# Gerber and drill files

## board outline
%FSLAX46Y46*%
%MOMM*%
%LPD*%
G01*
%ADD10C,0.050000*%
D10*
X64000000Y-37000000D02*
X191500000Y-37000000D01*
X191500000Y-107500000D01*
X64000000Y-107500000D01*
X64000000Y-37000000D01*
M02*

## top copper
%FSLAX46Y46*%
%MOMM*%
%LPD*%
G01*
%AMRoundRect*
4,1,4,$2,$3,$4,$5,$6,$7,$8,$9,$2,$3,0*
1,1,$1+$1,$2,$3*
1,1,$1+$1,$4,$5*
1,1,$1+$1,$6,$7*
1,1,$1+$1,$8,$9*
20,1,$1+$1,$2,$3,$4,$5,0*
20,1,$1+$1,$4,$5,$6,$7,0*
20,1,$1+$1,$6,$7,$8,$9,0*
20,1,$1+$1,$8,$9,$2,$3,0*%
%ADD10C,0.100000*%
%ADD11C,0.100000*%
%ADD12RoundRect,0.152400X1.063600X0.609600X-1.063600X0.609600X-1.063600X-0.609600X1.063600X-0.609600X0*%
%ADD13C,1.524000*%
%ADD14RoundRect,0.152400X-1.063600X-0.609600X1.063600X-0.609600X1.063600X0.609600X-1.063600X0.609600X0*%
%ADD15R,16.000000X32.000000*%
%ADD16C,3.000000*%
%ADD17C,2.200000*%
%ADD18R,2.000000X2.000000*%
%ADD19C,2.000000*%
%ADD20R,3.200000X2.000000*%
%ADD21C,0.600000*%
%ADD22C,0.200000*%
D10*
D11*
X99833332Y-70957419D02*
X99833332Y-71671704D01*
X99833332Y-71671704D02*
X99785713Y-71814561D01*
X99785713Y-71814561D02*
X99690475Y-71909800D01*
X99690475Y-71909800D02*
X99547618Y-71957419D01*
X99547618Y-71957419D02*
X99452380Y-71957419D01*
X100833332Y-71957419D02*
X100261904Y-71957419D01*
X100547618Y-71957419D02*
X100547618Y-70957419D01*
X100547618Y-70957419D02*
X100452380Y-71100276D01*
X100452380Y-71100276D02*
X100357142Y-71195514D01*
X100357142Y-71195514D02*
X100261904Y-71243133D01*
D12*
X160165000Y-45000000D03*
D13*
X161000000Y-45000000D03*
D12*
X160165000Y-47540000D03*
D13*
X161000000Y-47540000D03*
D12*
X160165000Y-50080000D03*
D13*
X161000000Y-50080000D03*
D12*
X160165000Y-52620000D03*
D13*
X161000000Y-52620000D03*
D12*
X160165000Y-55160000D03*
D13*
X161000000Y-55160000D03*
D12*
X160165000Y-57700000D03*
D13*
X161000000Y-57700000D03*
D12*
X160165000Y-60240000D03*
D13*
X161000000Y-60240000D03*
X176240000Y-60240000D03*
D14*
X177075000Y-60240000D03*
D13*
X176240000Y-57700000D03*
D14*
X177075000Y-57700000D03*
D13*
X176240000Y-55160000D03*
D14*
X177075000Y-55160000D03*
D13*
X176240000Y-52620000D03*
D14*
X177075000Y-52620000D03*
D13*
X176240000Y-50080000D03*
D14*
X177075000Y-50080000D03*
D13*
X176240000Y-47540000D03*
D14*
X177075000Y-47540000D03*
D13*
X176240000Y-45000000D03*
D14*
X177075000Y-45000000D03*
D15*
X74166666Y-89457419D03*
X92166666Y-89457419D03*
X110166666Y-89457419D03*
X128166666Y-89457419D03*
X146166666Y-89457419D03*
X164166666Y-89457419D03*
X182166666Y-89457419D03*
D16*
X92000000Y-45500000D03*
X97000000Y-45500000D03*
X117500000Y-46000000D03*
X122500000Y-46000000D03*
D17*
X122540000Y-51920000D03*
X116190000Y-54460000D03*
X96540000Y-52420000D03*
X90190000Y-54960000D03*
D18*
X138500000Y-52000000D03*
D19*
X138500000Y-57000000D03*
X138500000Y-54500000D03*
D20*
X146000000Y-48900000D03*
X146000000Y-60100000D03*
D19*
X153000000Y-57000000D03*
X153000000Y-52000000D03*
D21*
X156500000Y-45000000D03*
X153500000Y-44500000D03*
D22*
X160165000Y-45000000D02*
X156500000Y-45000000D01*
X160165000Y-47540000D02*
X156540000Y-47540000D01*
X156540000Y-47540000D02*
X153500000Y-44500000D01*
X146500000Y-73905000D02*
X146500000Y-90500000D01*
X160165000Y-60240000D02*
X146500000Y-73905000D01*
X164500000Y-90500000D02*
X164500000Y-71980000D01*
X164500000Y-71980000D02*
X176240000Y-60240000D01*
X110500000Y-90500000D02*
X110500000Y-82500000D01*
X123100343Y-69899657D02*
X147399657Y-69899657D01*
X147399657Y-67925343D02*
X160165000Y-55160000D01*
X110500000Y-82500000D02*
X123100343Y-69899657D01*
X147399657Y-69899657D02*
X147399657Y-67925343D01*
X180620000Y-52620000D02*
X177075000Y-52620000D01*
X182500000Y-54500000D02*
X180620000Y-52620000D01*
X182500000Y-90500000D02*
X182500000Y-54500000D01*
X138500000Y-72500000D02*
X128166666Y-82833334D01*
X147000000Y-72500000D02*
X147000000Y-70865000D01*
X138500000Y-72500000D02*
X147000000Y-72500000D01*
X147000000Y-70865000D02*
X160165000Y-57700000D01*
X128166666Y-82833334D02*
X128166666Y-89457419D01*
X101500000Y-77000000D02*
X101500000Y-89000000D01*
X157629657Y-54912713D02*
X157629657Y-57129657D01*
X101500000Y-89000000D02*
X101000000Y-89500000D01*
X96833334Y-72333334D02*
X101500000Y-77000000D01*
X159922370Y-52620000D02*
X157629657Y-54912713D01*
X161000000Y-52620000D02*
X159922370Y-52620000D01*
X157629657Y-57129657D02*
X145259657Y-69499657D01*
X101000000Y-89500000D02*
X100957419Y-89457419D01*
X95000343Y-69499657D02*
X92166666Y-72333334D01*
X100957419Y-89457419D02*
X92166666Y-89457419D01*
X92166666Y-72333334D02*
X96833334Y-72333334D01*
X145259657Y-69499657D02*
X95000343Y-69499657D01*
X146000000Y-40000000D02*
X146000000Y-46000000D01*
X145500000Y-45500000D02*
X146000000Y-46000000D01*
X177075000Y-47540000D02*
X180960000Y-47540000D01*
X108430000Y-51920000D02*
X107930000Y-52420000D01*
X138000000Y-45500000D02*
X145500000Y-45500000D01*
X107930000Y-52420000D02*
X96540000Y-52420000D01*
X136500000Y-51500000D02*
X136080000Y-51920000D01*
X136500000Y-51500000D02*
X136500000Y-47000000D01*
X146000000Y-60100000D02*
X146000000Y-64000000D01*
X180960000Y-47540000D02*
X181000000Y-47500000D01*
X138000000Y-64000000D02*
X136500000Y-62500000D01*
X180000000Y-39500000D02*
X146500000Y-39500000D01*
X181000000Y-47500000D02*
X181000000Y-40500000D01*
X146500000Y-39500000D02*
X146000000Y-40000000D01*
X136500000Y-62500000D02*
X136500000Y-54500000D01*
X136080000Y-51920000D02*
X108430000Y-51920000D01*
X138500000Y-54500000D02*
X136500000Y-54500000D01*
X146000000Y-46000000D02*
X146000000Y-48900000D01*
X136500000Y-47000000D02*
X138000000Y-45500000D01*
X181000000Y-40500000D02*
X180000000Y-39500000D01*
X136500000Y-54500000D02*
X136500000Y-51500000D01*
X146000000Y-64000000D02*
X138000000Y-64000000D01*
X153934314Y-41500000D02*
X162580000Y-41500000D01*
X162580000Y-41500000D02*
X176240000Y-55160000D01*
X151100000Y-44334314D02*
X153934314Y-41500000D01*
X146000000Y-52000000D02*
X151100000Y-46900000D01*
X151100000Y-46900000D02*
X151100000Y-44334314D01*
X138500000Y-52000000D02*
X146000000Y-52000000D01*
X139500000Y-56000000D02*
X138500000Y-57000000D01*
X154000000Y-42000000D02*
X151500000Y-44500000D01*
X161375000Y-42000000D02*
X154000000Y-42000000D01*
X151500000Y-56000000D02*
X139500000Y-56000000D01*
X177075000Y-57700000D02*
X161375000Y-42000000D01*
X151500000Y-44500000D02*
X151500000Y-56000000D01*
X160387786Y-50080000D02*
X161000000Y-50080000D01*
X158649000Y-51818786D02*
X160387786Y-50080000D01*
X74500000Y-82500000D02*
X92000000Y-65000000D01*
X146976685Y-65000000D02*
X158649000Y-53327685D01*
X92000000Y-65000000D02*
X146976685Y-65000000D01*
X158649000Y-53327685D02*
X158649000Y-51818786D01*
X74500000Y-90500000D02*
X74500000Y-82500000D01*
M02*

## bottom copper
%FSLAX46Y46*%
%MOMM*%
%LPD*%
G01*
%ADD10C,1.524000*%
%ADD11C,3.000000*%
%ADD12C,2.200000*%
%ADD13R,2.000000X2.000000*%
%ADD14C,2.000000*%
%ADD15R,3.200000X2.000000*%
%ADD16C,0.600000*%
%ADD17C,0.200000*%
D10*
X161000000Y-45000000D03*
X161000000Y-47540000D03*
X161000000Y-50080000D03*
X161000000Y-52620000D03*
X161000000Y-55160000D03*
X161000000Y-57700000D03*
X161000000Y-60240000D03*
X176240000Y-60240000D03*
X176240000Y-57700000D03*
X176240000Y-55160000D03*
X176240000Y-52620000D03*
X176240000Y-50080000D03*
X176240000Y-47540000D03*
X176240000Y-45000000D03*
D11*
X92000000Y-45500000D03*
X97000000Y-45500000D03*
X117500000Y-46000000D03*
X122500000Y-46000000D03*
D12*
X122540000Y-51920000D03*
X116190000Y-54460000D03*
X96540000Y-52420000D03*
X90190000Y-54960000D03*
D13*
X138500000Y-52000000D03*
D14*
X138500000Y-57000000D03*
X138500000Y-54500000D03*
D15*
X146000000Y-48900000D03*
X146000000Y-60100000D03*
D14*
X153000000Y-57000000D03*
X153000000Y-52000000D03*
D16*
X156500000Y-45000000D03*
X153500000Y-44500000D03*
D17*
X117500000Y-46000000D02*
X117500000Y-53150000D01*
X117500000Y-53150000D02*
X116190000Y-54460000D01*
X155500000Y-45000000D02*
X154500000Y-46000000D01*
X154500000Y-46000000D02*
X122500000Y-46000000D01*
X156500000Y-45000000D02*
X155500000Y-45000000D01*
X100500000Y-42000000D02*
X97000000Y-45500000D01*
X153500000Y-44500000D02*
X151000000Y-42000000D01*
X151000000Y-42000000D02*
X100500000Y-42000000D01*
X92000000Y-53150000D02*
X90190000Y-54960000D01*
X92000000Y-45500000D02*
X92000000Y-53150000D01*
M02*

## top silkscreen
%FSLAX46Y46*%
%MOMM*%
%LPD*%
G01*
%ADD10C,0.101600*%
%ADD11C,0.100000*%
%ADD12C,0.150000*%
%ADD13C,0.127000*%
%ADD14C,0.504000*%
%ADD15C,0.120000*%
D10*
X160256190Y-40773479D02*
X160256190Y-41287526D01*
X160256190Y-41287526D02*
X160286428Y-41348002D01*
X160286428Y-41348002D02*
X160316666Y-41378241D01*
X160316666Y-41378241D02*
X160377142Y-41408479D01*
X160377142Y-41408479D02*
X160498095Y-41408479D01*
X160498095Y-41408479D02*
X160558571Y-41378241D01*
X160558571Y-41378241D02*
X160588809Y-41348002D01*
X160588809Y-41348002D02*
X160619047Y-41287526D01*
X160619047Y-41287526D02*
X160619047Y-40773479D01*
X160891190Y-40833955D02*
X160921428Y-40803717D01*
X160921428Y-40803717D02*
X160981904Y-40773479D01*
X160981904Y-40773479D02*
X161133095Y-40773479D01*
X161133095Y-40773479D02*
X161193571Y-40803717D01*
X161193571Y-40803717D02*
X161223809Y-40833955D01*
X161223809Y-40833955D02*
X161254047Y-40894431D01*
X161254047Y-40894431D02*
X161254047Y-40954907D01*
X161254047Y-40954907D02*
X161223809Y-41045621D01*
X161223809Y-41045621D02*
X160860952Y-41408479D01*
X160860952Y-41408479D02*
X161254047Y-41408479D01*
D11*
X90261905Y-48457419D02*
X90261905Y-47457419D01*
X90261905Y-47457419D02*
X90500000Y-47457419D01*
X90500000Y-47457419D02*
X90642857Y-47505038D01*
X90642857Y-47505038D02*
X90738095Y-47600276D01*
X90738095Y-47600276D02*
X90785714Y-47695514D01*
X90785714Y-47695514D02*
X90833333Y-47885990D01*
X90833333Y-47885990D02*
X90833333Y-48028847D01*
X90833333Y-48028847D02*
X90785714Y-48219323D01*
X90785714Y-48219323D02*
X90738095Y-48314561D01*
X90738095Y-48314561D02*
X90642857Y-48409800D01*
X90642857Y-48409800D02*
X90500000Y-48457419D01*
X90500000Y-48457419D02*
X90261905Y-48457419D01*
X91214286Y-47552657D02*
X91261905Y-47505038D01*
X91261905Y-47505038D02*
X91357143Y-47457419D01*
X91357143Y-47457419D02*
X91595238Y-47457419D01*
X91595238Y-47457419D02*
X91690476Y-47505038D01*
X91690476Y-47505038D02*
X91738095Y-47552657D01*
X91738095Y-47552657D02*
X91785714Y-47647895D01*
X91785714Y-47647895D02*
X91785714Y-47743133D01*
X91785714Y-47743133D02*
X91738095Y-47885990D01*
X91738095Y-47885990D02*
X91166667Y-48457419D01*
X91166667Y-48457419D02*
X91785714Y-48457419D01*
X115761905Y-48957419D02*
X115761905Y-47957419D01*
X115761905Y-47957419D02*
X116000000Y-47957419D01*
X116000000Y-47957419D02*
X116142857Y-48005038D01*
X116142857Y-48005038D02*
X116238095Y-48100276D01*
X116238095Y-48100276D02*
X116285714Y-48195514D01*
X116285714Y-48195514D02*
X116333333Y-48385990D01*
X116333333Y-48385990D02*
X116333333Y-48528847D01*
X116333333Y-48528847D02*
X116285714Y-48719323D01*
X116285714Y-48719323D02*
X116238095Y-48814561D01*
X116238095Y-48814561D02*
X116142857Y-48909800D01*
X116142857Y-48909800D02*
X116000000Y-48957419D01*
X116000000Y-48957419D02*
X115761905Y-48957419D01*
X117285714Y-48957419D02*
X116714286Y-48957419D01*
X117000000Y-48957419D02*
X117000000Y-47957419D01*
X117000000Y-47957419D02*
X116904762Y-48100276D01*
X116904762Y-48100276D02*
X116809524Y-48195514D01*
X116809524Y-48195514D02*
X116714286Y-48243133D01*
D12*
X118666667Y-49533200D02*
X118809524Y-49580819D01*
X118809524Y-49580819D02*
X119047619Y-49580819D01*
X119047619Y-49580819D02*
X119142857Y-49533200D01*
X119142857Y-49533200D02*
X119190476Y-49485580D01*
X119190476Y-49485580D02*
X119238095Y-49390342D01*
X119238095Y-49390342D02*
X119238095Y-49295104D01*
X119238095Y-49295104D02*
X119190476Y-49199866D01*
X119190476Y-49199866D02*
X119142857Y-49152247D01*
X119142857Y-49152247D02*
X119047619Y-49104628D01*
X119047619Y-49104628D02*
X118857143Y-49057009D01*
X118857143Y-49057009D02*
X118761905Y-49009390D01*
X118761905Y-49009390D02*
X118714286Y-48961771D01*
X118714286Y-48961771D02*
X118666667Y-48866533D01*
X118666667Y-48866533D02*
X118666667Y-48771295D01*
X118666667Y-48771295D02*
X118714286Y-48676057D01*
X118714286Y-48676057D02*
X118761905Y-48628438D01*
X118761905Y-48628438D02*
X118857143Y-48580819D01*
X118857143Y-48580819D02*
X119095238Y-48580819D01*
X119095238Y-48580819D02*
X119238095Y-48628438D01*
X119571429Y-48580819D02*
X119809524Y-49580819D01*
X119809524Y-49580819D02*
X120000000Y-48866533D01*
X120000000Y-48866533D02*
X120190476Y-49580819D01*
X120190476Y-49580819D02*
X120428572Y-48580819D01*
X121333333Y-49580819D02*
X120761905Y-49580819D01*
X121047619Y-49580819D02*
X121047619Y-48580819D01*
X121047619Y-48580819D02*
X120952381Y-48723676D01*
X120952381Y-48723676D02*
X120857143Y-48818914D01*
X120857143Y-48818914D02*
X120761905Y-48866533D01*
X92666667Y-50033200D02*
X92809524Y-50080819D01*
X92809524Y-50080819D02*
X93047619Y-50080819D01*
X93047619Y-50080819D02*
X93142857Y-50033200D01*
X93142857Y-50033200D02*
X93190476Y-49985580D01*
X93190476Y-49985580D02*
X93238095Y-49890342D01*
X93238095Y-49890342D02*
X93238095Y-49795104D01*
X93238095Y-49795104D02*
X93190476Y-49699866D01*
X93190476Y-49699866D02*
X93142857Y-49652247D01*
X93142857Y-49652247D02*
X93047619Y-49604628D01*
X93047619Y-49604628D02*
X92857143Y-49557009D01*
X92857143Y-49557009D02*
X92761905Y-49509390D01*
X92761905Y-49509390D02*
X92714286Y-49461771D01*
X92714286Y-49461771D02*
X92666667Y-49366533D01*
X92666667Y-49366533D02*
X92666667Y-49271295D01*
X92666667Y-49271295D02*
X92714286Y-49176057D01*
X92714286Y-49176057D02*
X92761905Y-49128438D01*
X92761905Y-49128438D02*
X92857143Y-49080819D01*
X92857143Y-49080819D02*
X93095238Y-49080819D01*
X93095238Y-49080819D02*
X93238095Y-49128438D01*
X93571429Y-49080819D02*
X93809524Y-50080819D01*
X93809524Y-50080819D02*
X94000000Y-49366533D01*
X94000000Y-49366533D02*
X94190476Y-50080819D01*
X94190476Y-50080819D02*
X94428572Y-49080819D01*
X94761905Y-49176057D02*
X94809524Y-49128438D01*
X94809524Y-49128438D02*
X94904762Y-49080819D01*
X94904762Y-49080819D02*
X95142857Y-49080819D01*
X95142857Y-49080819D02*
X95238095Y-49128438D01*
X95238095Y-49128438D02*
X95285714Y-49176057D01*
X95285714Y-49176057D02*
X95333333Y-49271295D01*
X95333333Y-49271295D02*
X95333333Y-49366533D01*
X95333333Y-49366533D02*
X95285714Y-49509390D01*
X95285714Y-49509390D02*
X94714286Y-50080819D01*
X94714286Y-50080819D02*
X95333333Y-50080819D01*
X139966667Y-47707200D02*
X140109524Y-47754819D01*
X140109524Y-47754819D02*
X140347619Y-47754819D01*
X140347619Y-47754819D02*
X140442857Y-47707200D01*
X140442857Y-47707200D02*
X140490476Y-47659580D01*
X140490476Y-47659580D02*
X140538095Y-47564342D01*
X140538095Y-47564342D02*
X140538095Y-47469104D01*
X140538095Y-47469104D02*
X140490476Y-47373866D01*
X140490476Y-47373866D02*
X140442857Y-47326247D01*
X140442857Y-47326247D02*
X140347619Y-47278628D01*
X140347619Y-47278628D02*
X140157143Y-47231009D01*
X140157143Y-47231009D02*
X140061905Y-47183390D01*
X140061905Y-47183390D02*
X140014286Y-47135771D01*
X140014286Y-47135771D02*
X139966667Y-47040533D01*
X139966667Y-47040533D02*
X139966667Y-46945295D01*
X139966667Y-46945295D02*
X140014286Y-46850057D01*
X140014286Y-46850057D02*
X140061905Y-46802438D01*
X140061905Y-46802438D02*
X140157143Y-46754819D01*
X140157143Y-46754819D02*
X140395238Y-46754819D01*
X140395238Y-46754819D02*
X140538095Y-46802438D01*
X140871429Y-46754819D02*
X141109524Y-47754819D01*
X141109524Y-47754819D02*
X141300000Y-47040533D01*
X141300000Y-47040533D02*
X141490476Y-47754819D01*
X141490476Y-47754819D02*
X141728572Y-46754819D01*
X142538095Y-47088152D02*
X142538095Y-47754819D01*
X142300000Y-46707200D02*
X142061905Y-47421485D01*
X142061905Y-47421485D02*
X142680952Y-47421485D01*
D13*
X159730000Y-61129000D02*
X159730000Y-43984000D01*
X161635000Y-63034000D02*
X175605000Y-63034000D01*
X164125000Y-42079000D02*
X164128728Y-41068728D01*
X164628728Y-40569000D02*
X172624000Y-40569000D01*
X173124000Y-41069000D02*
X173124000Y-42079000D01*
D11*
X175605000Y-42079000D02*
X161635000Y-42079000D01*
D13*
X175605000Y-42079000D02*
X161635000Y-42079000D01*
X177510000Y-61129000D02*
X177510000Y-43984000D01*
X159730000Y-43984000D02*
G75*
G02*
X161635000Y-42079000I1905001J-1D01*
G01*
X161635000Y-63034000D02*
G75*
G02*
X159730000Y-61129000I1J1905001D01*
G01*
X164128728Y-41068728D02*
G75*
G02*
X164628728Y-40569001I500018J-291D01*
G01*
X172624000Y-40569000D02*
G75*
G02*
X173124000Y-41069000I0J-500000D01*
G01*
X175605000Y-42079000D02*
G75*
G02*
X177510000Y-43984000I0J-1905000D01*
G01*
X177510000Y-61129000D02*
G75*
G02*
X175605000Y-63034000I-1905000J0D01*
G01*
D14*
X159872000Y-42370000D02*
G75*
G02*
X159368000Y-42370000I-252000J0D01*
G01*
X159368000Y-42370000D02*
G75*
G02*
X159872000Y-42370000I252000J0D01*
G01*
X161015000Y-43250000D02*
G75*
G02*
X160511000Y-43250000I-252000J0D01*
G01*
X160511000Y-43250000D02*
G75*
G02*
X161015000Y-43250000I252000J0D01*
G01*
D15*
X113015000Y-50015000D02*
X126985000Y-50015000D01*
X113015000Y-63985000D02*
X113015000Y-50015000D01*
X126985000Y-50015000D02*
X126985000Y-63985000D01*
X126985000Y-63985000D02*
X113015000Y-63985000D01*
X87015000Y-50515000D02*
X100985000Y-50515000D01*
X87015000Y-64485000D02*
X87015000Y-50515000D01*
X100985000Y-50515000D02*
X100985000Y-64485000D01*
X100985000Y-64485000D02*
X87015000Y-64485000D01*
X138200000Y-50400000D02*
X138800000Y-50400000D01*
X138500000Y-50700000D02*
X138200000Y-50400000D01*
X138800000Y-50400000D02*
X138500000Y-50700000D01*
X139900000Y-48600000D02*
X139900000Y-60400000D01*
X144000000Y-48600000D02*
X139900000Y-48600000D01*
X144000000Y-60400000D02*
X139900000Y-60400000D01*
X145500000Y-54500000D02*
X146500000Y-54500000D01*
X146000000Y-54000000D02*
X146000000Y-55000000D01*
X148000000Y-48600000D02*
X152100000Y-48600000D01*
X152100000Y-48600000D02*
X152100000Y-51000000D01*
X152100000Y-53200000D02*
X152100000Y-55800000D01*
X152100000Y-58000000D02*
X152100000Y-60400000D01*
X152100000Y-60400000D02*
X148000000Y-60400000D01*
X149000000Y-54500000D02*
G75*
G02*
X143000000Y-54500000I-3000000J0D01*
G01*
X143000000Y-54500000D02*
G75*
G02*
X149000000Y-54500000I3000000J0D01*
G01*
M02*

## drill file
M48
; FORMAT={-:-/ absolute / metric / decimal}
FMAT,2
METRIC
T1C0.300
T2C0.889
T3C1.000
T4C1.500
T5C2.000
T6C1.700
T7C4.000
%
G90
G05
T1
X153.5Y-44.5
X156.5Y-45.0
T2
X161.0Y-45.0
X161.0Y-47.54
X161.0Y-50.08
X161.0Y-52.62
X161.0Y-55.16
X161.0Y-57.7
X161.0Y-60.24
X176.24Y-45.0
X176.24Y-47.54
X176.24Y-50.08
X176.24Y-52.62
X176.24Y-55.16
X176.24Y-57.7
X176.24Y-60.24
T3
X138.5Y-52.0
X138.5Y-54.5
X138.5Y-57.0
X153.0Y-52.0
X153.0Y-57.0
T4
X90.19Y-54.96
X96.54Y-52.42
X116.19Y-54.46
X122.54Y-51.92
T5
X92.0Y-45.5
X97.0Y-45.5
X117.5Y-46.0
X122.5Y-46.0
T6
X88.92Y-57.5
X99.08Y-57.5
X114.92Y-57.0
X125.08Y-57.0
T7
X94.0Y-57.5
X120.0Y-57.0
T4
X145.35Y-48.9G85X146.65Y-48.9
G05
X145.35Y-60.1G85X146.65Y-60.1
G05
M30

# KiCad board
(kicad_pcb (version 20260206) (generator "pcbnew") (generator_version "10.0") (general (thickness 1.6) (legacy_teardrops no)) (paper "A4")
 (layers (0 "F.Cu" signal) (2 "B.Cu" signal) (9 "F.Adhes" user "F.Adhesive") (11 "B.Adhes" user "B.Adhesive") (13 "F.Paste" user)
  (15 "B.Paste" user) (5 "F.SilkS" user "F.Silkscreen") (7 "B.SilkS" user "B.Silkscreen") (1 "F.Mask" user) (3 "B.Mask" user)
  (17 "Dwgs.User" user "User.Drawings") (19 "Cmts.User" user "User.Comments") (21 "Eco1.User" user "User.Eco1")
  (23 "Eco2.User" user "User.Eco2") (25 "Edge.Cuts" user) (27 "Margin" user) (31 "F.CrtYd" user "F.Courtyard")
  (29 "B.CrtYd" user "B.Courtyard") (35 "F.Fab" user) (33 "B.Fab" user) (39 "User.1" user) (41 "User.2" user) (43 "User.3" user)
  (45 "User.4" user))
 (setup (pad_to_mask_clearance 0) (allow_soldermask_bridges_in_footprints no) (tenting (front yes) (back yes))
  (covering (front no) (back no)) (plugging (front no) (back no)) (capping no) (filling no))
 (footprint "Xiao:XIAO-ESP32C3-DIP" (layer "F.Cu") (at 168.74 52.62)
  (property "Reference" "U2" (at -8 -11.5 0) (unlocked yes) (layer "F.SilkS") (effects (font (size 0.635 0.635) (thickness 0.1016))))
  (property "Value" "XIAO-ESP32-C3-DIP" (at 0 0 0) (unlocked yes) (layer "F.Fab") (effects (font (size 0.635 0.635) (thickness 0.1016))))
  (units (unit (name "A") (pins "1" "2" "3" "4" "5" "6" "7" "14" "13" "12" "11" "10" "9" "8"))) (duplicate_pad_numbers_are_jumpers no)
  (fp_line (start -9.01 8.509) (end -9.01 -8.636) (stroke (width 0.127) (type solid)) (layer "F.SilkS"))
  (fp_line (start -7.105 10.414) (end 6.865 10.414) (stroke (width 0.127) (type solid)) (layer "F.SilkS"))
  (fp_line (start -4.615 -10.541) (end -4.611272 -11.551272) (stroke (width 0.127) (type solid)) (layer "F.SilkS"))
  (fp_line (start -4.111272 -12.051) (end 3.884 -12.051) (stroke (width 0.127) (type solid)) (layer "F.SilkS"))
  (fp_line (start 4.384 -11.551) (end 4.384 -10.541) (stroke (width 0.127) (type solid)) (layer "F.SilkS"))
  (fp_line (start 6.865 -10.541) (end -7.105 -10.541) (stroke (width 0.1) (type solid)) (layer "F.SilkS"))
  (fp_line (start 6.865 -10.541) (end -7.105 -10.541) (stroke (width 0.127) (type solid)) (layer "F.SilkS"))
  (fp_line (start 8.77 8.509) (end 8.77 -8.636) (stroke (width 0.127) (type solid)) (layer "F.SilkS"))
  (fp_arc (start -9.01 -8.636) (mid -8.452038 -9.983038) (end -7.105 -10.541) (stroke (width 0.127) (type solid)) (layer "F.SilkS"))
  (fp_arc (start -7.105 10.414) (mid -8.452038 9.856038) (end -9.01 8.509) (stroke (width 0.127) (type solid)) (layer "F.SilkS"))
  (fp_arc (start -4.611272 -11.551272) (mid -4.464728 -11.90464) (end -4.111272 -12.051) (stroke (width 0.127) (type default))
   (layer "F.SilkS"))
  (fp_arc (start 3.884 -12.051) (mid 4.237553 -11.904553) (end 4.384 -11.551) (stroke (width 0.127) (type default)) (layer "F.SilkS"))
  (fp_arc (start 6.865 -10.541) (mid 8.212038 -9.983038) (end 8.77 -8.636) (stroke (width 0.127) (type solid)) (layer "F.SilkS"))
  (fp_arc (start 8.77 8.509) (mid 8.212038 9.856038) (end 6.865 10.414) (stroke (width 0.127) (type solid)) (layer "F.SilkS"))
  (fp_circle (center -9.12 -10.25) (end -9.12 -10.504) (stroke (width 0.5) (type solid)) (fill yes) (layer "F.SilkS"))
  (fp_circle (center -7.977 -9.37) (end -7.977 -9.624) (stroke (width 0.5) (type solid)) (fill yes) (layer "F.SilkS"))
  (pad "1" smd roundrect (at -8.575 -7.62 180) (size 2.432 1.524) (layers "F.Cu" "F.Mask") (roundrect_rratio 0.1) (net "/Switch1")
   (thermal_bridge_angle 45))
  (pad "1" thru_hole circle (at -7.74 -7.62 180) (size 1.524 1.524) (drill 0.889) (layers "*.Cu" "*.Mask") (remove_unused_layers no)
   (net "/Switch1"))
  (pad "2" smd roundrect (at -8.575 -5.08 180) (size 2.432 1.524) (layers "F.Cu" "F.Mask") (roundrect_rratio 0.1) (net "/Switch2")
   (thermal_bridge_angle 45))
  (pad "2" thru_hole circle (at -7.74 -5.08 180) (size 1.524 1.524) (drill 0.889) (layers "*.Cu" "*.Mask") (remove_unused_layers no)
   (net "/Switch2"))
  (pad "3" smd roundrect (at -8.575 -2.54 180) (size 2.432 1.524) (layers "F.Cu" "F.Mask") (roundrect_rratio 0.1) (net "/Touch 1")
   (thermal_bridge_angle 45))
  (pad "3" thru_hole circle (at -7.74 -2.54 180) (size 1.524 1.524) (drill 0.889) (layers "*.Cu" "*.Mask") (remove_unused_layers no)
   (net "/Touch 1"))
  (pad "4" smd roundrect (at -8.575 0 180) (size 2.432 1.524) (layers "F.Cu" "F.Mask") (roundrect_rratio 0.1) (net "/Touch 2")
   (thermal_bridge_angle 45))
  (pad "4" thru_hole circle (at -7.74 0 180) (size 1.524 1.524) (drill 0.889) (layers "*.Cu" "*.Mask") (remove_unused_layers no)
   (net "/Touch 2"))
  (pad "5" smd roundrect (at -8.575 2.54 180) (size 2.432 1.524) (layers "F.Cu" "F.Mask") (roundrect_rratio 0.1) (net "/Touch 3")
   (thermal_bridge_angle 45))
  (pad "5" thru_hole circle (at -7.74 2.54 180) (size 1.524 1.524) (drill 0.889) (layers "*.Cu" "*.Mask") (remove_unused_layers no)
   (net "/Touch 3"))
  (pad "6" smd roundrect (at -8.575 5.08 180) (size 2.432 1.524) (layers "F.Cu" "F.Mask") (roundrect_rratio 0.1) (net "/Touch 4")
   (thermal_bridge_angle 45))
  (pad "6" thru_hole circle (at -7.74 5.08 180) (size 1.524 1.524) (drill 0.889) (layers "*.Cu" "*.Mask") (remove_unused_layers no)
   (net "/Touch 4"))
  (pad "7" smd roundrect (at -8.575 7.62 180) (size 2.432 1.524) (layers "F.Cu" "F.Mask") (roundrect_rratio 0.1) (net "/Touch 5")
   (thermal_bridge_angle 45))
  (pad "7" thru_hole circle (at -7.74 7.62 180) (size 1.524 1.524) (drill 0.889) (layers "*.Cu" "*.Mask") (remove_unused_layers no)
   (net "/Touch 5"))
  (pad "8" thru_hole circle (at 7.5 7.62) (size 1.524 1.524) (drill 0.889) (layers "*.Cu" "*.Mask") (remove_unused_layers no)
   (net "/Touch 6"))
  (pad "8" smd roundrect (at 8.335 7.62) (size 2.432 1.524) (layers "F.Cu" "F.Mask") (roundrect_rratio 0.1) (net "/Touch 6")
   (thermal_bridge_angle 45))
  (pad "9" thru_hole circle (at 7.5 5.08) (size 1.524 1.524) (drill 0.889) (layers "*.Cu" "*.Mask") (remove_unused_layers no)
   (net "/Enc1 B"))
  (pad "9" smd roundrect (at 8.335 5.08) (size 2.432 1.524) (layers "F.Cu" "F.Mask") (roundrect_rratio 0.1) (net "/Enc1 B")
   (thermal_bridge_angle 45))
  (pad "10" thru_hole circle (at 7.5 2.54) (size 1.524 1.524) (drill 0.889) (layers "*.Cu" "*.Mask") (remove_unused_layers no)
   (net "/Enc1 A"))
  (pad "10" smd roundrect (at 8.335 2.54) (size 2.432 1.524) (layers "F.Cu" "F.Mask") (roundrect_rratio 0.1) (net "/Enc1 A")
   (thermal_bridge_angle 45))
  (pad "11" thru_hole circle (at 7.5 0) (size 1.524 1.524) (drill 0.889) (layers "*.Cu" "*.Mask") (remove_unused_layers no) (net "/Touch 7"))
  (pad "11" smd roundrect (at 8.335 0) (size 2.432 1.524) (layers "F.Cu" "F.Mask") (roundrect_rratio 0.1) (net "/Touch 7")
   (thermal_bridge_angle 45))
  (pad "12" thru_hole circle (at 7.5 -2.54) (size 1.524 1.524) (drill 0.889) (layers "*.Cu" "*.Mask") (remove_unused_layers no) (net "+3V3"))
  (pad "12" smd roundrect (at 8.335 -2.54) (size 2.432 1.524) (layers "F.Cu" "F.Mask") (roundrect_rratio 0.1) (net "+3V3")
   (thermal_bridge_angle 45))
  (pad "13" thru_hole circle (at 7.5 -5.08) (size 1.524 1.524) (drill 0.889) (layers "*.Cu" "*.Mask") (remove_unused_layers no) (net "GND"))
  (pad "13" smd roundrect (at 8.335 -5.08) (size 2.432 1.524) (layers "F.Cu" "F.Mask") (roundrect_rratio 0.1) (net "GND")
   (thermal_bridge_angle 45))
  (pad "14" thru_hole circle (at 7.5 -7.62) (size 1.524 1.524) (drill 0.889) (layers "*.Cu" "*.Mask") (remove_unused_layers no)
   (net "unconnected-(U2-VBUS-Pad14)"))
  (pad "14" smd roundrect (at 8.335 -7.62) (size 2.432 1.524) (layers "F.Cu" "F.Mask") (roundrect_rratio 0.1)
   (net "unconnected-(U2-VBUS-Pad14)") (thermal_bridge_angle 45)))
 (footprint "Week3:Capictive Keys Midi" (layer "F.Cu") (at 93.166666 89.457419)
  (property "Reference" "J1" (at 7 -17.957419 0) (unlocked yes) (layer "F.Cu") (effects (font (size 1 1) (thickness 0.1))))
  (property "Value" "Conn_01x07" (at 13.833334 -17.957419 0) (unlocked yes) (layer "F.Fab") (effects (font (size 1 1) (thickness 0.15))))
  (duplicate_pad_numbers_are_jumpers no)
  (pad "1" smd rect (at -19 0) (size 16 32) (layers "F.Cu" "F.Mask") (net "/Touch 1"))
  (pad "2" smd rect (at -1 0) (size 16 32) (layers "F.Cu" "F.Mask") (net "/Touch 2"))
  (pad "3" smd rect (at 17 0) (size 16 32) (layers "F.Cu" "F.Mask") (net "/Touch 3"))
  (pad "4" smd rect (at 35 0) (size 16 32) (layers "F.Cu" "F.Mask") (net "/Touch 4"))
  (pad "5" smd rect (at 53 0) (size 16 32) (layers "F.Cu" "F.Mask") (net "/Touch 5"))
  (pad "6" smd rect (at 71 0) (size 16 32) (layers "F.Cu" "F.Mask") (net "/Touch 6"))
  (pad "7" smd rect (at 89 0) (size 16 32) (layers "F.Cu" "F.Mask") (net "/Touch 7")))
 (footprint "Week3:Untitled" (layer "F.Cu") (at 91 48.5)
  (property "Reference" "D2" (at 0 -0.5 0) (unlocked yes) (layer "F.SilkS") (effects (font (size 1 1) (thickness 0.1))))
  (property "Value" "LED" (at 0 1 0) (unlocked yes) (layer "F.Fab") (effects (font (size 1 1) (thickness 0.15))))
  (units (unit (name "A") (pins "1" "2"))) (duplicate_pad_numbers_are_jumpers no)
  (pad "1" thru_hole circle (at 1 -3) (size 3 3) (drill 2) (layers "*.Cu" "*.Mask") (remove_unused_layers no) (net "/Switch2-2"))
  (pad "2" thru_hole circle (at 6 -3) (size 3 3) (drill 2) (layers "*.Cu" "*.Mask") (remove_unused_layers no) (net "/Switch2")))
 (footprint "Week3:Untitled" (layer "F.Cu") (at 116.5 49)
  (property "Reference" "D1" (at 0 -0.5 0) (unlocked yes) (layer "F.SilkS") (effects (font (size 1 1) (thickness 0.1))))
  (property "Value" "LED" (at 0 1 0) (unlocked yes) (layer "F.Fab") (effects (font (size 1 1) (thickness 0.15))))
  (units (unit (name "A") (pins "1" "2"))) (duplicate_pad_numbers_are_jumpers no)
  (pad "1" thru_hole circle (at 1 -3) (size 3 3) (drill 2) (layers "*.Cu" "*.Mask") (remove_unused_layers no) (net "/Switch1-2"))
  (pad "2" thru_hole circle (at 6 -3) (size 3 3) (drill 2) (layers "*.Cu" "*.Mask") (remove_unused_layers no) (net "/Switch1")))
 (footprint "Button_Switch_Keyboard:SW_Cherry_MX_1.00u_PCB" (layer "F.Cu") (at 122.54 51.92)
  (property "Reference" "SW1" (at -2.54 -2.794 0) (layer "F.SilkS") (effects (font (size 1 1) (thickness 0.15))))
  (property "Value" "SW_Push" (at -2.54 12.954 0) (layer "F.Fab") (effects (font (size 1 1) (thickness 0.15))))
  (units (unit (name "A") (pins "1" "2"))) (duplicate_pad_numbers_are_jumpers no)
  (fp_line (start -9.525 -1.905) (end 4.445 -1.905) (stroke (width 0.12) (type solid)) (layer "F.SilkS"))
  (fp_line (start -9.525 12.065) (end -9.525 -1.905) (stroke (width 0.12) (type solid)) (layer "F.SilkS"))
  (fp_line (start 4.445 -1.905) (end 4.445 12.065) (stroke (width 0.12) (type solid)) (layer "F.SilkS"))
  (fp_line (start 4.445 12.065) (end -9.525 12.065) (stroke (width 0.12) (type solid)) (layer "F.SilkS"))
  (pad "" np_thru_hole circle (at -7.62 5.08) (size 1.7 1.7) (drill 1.7) (layers "*.Cu" "*.Mask"))
  (pad "" np_thru_hole circle (at -2.54 5.08) (size 4 4) (drill 4) (layers "*.Cu" "*.Mask"))
  (pad "" np_thru_hole circle (at 2.54 5.08) (size 1.7 1.7) (drill 1.7) (layers "*.Cu" "*.Mask"))
  (pad "1" thru_hole circle (at 0 0) (size 2.2 2.2) (drill 1.5) (layers "*.Cu" "*.Mask") (remove_unused_layers no) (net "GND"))
  (pad "2" thru_hole circle (at -6.35 2.54) (size 2.2 2.2) (drill 1.5) (layers "*.Cu" "*.Mask") (remove_unused_layers no) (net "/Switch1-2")))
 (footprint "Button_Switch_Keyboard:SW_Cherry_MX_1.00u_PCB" (layer "F.Cu") (at 96.54 52.42)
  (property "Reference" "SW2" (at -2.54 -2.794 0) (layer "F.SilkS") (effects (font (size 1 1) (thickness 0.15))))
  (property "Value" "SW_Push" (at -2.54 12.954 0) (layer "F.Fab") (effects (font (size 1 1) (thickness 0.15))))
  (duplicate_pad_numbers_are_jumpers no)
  (fp_line (start -9.525 -1.905) (end 4.445 -1.905) (stroke (width 0.12) (type solid)) (layer "F.SilkS"))
  (fp_line (start -9.525 12.065) (end -9.525 -1.905) (stroke (width 0.12) (type solid)) (layer "F.SilkS"))
  (fp_line (start 4.445 -1.905) (end 4.445 12.065) (stroke (width 0.12) (type solid)) (layer "F.SilkS"))
  (fp_line (start 4.445 12.065) (end -9.525 12.065) (stroke (width 0.12) (type solid)) (layer "F.SilkS"))
  (pad "" np_thru_hole circle (at -7.62 5.08) (size 1.7 1.7) (drill 1.7) (layers "*.Cu" "*.Mask"))
  (pad "" np_thru_hole circle (at -2.54 5.08) (size 4 4) (drill 4) (layers "*.Cu" "*.Mask"))
  (pad "" np_thru_hole circle (at 2.54 5.08) (size 1.7 1.7) (drill 1.7) (layers "*.Cu" "*.Mask"))
  (pad "1" thru_hole circle (at 0 0) (size 2.2 2.2) (drill 1.5) (layers "*.Cu" "*.Mask") (remove_unused_layers no) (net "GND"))
  (pad "2" thru_hole circle (at -6.35 2.54) (size 2.2 2.2) (drill 1.5) (layers "*.Cu" "*.Mask") (remove_unused_layers no) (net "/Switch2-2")))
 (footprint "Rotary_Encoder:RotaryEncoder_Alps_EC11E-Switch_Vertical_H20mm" (layer "F.Cu") (at 138.5 52)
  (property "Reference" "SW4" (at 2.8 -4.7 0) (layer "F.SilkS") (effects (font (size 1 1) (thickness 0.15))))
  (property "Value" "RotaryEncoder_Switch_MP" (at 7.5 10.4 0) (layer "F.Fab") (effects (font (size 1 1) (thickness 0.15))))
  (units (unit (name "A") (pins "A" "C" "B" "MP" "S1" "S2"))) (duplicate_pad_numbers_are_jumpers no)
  (fp_line (start -0.3 -1.6) (end 0.3 -1.6) (stroke (width 0.12) (type solid)) (layer "F.SilkS"))
  (fp_line (start 0 -1.3) (end -0.3 -1.6) (stroke (width 0.12) (type solid)) (layer "F.SilkS"))
  (fp_line (start 0.3 -1.6) (end 0 -1.3) (stroke (width 0.12) (type solid)) (layer "F.SilkS"))
  (fp_line (start 1.4 -3.4) (end 1.4 8.4) (stroke (width 0.12) (type solid)) (layer "F.SilkS"))
  (fp_line (start 5.5 -3.4) (end 1.4 -3.4) (stroke (width 0.12) (type solid)) (layer "F.SilkS"))
  (fp_line (start 5.5 8.4) (end 1.4 8.4) (stroke (width 0.12) (type solid)) (layer "F.SilkS"))
  (fp_line (start 7 2.5) (end 8 2.5) (stroke (width 0.12) (type solid)) (layer "F.SilkS"))
  (fp_line (start 7.5 2) (end 7.5 3) (stroke (width 0.12) (type solid)) (layer "F.SilkS"))
  (fp_line (start 9.5 -3.4) (end 13.6 -3.4) (stroke (width 0.12) (type solid)) (layer "F.SilkS"))
  (fp_line (start 13.6 -3.4) (end 13.6 -1) (stroke (width 0.12) (type solid)) (layer "F.SilkS"))
  (fp_line (start 13.6 1.2) (end 13.6 3.8) (stroke (width 0.12) (type solid)) (layer "F.SilkS"))
  (fp_line (start 13.6 6) (end 13.6 8.4) (stroke (width 0.12) (type solid)) (layer "F.SilkS"))
  (fp_line (start 13.6 8.4) (end 9.5 8.4) (stroke (width 0.12) (type solid)) (layer "F.SilkS"))
  (fp_circle (center 7.5 2.5) (end 10.5 2.5) (stroke (width 0.12) (type solid)) (fill no) (layer "F.SilkS"))
  (pad "A" thru_hole rect (at 0 0) (size 2 2) (drill 1) (layers "*.Cu" "*.Mask") (remove_unused_layers no) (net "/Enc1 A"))
  (pad "B" thru_hole circle (at 0 5) (size 2 2) (drill 1) (layers "*.Cu" "*.Mask") (remove_unused_layers no) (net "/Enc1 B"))
  (pad "C" thru_hole circle (at 0 2.5) (size 2 2) (drill 1) (layers "*.Cu" "*.Mask") (remove_unused_layers no) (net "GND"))
  (pad "MP" thru_hole rect (at 7.5 -3.1) (size 3.2 2) (drill oval 2.8 1.5) (layers "*.Cu" "*.Mask") (remove_unused_layers no) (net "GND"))
  (pad "MP" thru_hole rect (at 7.5 8.1) (size 3.2 2) (drill oval 2.8 1.5) (layers "*.Cu" "*.Mask") (remove_unused_layers no) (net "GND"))
  (pad "S1" thru_hole circle (at 14.5 5) (size 2 2) (drill 1) (layers "*.Cu" "*.Mask") (remove_unused_layers no)
   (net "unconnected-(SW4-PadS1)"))
  (pad "S2" thru_hole circle (at 14.5 0) (size 2 2) (drill 1) (layers "*.Cu" "*.Mask") (remove_unused_layers no)
   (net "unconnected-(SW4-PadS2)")))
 (gr_rect (start 64 37) (end 191.5 107.5) (stroke (width 0.05) (type default)) (fill no) (layer "Edge.Cuts"))
 (segment (start 117.5 46) (end 117.5 53.15) (width 0.2) (layer "B.Cu") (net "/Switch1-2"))
 (segment (start 117.5 53.15) (end 116.19 54.46) (width 0.2) (layer "B.Cu") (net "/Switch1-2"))
 (segment (start 160.165 45) (end 156.5 45) (width 0.2) (layer "F.Cu") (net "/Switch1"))
 (via blind (at 156.5 45) (size 0.6) (drill 0.3) (layers "F.Cu" "B.Cu") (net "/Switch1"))
 (segment (start 155.5 45) (end 154.5 46) (width 0.2) (layer "B.Cu") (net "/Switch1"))
 (segment (start 154.5 46) (end 122.5 46) (width 0.2) (layer "B.Cu") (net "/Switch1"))
 (segment (start 156.5 45) (end 155.5 45) (width 0.2) (layer "B.Cu") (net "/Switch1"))
 (segment (start 160.165 47.54) (end 156.54 47.54) (width 0.2) (layer "F.Cu") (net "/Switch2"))
 (segment (start 156.54 47.54) (end 153.5 44.5) (width 0.2) (layer "F.Cu") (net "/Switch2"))
 (via blind (at 153.5 44.5) (size 0.6) (drill 0.3) (layers "F.Cu" "B.Cu") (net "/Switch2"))
 (segment (start 100.5 42) (end 97 45.5) (width 0.2) (layer "B.Cu") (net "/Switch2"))
 (segment (start 153.5 44.5) (end 151 42) (width 0.2) (layer "B.Cu") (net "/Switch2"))
 (segment (start 151 42) (end 100.5 42) (width 0.2) (layer "B.Cu") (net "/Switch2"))
 (segment (start 92 53.15) (end 90.19 54.96) (width 0.2) (layer "B.Cu") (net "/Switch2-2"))
 (segment (start 92 45.5) (end 92 53.15) (width 0.2) (layer "B.Cu") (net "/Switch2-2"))
 (segment (start 146.5 73.905) (end 146.5 90.5) (width 0.2) (layer "F.Cu") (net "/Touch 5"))
 (segment (start 160.165 60.24) (end 146.5 73.905) (width 0.2) (layer "F.Cu") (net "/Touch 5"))
 (segment (start 164.5 90.5) (end 164.5 71.98) (width 0.2) (layer "F.Cu") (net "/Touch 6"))
 (segment (start 164.5 71.98) (end 176.24 60.24) (width 0.2) (layer "F.Cu") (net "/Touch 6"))
 (segment (start 110.5 90.5) (end 110.5 82.5) (width 0.2) (layer "F.Cu") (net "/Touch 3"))
 (segment (start 123.100343 69.899657) (end 147.399657 69.899657) (width 0.2) (layer "F.Cu") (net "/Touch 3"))
 (segment (start 147.399657 67.925343) (end 160.165 55.16) (width 0.2) (layer "F.Cu") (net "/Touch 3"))
 (segment (start 110.5 82.5) (end 123.100343 69.899657) (width 0.2) (layer "F.Cu") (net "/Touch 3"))
 (segment (start 147.399657 69.899657) (end 147.399657 67.925343) (width 0.2) (layer "F.Cu") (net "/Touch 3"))
 (segment (start 180.62 52.62) (end 177.075 52.62) (width 0.2) (layer "F.Cu") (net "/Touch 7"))
 (segment (start 182.5 54.5) (end 180.62 52.62) (width 0.2) (layer "F.Cu") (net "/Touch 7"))
 (segment (start 182.5 90.5) (end 182.5 54.5) (width 0.2) (layer "F.Cu") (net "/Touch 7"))
 (segment (start 138.5 72.5) (end 128.166666 82.833334) (width 0.2) (layer "F.Cu") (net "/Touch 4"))
 (segment (start 147 72.5) (end 147 70.865) (width 0.2) (layer "F.Cu") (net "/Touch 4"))
 (segment (start 138.5 72.5) (end 147 72.5) (width 0.2) (layer "F.Cu") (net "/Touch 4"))
 (segment (start 147 70.865) (end 160.165 57.7) (width 0.2) (layer "F.Cu") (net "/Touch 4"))
 (segment (start 128.166666 82.833334) (end 128.166666 89.457419) (width 0.2) (layer "F.Cu") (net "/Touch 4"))
 (segment (start 101.5 77) (end 101.5 89) (width 0.2) (layer "F.Cu") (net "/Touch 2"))
 (segment (start 157.629657 54.912713) (end 157.629657 57.129657) (width 0.2) (layer "F.Cu") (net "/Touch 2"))
 (segment (start 101.5 89) (end 101 89.5) (width 0.2) (layer "F.Cu") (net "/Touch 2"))
 (segment (start 96.833334 72.333334) (end 101.5 77) (width 0.2) (layer "F.Cu") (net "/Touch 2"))
 (segment (start 159.92237 52.62) (end 157.629657 54.912713) (width 0.2) (layer "F.Cu") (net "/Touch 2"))
 (segment (start 161 52.62) (end 159.92237 52.62) (width 0.2) (layer "F.Cu") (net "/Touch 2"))
 (segment (start 157.629657 57.129657) (end 145.259657 69.499657) (width 0.2) (layer "F.Cu") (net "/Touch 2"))
 (segment (start 101 89.5) (end 100.957419 89.457419) (width 0.2) (layer "F.Cu") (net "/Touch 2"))
 (segment (start 95.000343 69.499657) (end 92.166666 72.333334) (width 0.2) (layer "F.Cu") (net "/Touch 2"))
 (segment (start 100.957419 89.457419) (end 92.166666 89.457419) (width 0.2) (layer "F.Cu") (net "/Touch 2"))
 (segment (start 92.166666 72.333334) (end 96.833334 72.333334) (width 0.2) (layer "F.Cu") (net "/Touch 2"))
 (segment (start 145.259657 69.499657) (end 95.000343 69.499657) (width 0.2) (layer "F.Cu") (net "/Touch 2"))
 (segment (start 146 40) (end 146 46) (width 0.2) (layer "F.Cu") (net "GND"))
 (segment (start 145.5 45.5) (end 146 46) (width 0.2) (layer "F.Cu") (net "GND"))
 (segment (start 177.075 47.54) (end 180.96 47.54) (width 0.2) (layer "F.Cu") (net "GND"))
 (segment (start 108.43 51.92) (end 107.93 52.42) (width 0.2) (layer "F.Cu") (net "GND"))
 (segment (start 138 45.5) (end 145.5 45.5) (width 0.2) (layer "F.Cu") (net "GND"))
 (segment (start 107.93 52.42) (end 96.54 52.42) (width 0.2) (layer "F.Cu") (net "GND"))
 (segment (start 136.5 51.5) (end 136.08 51.92) (width 0.2) (layer "F.Cu") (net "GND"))
 (segment (start 136.5 51.5) (end 136.5 47) (width 0.2) (layer "F.Cu") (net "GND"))
 (segment (start 146 60.1) (end 146 64) (width 0.2) (layer "F.Cu") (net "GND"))
 (segment (start 180.96 47.54) (end 181 47.5) (width 0.2) (layer "F.Cu") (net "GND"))
 (segment (start 138 64) (end 136.5 62.5) (width 0.2) (layer "F.Cu") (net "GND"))
 (segment (start 180 39.5) (end 146.5 39.5) (width 0.2) (layer "F.Cu") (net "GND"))
 (segment (start 181 47.5) (end 181 40.5) (width 0.2) (layer "F.Cu") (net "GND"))
 (segment (start 146.5 39.5) (end 146 40) (width 0.2) (layer "F.Cu") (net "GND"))
 (segment (start 136.5 62.5) (end 136.5 54.5) (width 0.2) (layer "F.Cu") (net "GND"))
 (segment (start 136.08 51.92) (end 108.43 51.92) (width 0.2) (layer "F.Cu") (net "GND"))
 (segment (start 138.5 54.5) (end 136.5 54.5) (width 0.2) (layer "F.Cu") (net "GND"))
 (segment (start 146 46) (end 146 48.9) (width 0.2) (layer "F.Cu") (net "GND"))
 (segment (start 136.5 47) (end 138 45.5) (width 0.2) (layer "F.Cu") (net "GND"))
 (segment (start 181 40.5) (end 180 39.5) (width 0.2) (layer "F.Cu") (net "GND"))
 (segment (start 136.5 54.5) (end 136.5 51.5) (width 0.2) (layer "F.Cu") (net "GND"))
 (segment (start 146 64) (end 138 64) (width 0.2) (layer "F.Cu") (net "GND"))
 (segment (start 153.934314 41.5) (end 162.58 41.5) (width 0.2) (layer "F.Cu") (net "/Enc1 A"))
 (segment (start 162.58 41.5) (end 176.24 55.16) (width 0.2) (layer "F.Cu") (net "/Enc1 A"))
 (segment (start 151.1 44.334314) (end 153.934314 41.5) (width 0.2) (layer "F.Cu") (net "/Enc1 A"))
 (segment (start 146 52) (end 151.1 46.9) (width 0.2) (layer "F.Cu") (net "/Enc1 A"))
 (segment (start 151.1 46.9) (end 151.1 44.334314) (width 0.2) (layer "F.Cu") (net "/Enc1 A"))
 (segment (start 138.5 52) (end 146 52) (width 0.2) (layer "F.Cu") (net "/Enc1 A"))
 (segment (start 139.5 56) (end 138.5 57) (width 0.2) (layer "F.Cu") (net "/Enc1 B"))
 (segment (start 154 42) (end 151.5 44.5) (width 0.2) (layer "F.Cu") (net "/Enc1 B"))
 (segment (start 161.375 42) (end 154 42) (width 0.2) (layer "F.Cu") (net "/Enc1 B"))
 (segment (start 151.5 56) (end 139.5 56) (width 0.2) (layer "F.Cu") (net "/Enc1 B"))
 (segment (start 177.075 57.7) (end 161.375 42) (width 0.2) (layer "F.Cu") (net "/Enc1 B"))
 (segment (start 151.5 44.5) (end 151.5 56) (width 0.2) (layer "F.Cu") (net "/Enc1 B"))
 (segment (start 160.387786 50.08) (end 161 50.08) (width 0.2) (layer "F.Cu") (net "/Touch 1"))
 (segment (start 158.649 51.818786) (end 160.387786 50.08) (width 0.2) (layer "F.Cu") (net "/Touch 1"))
 (segment (start 74.5 82.5) (end 92 65) (width 0.2) (layer "F.Cu") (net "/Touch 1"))
 (segment (start 146.976685 65) (end 158.649 53.327685) (width 0.2) (layer "F.Cu") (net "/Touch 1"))
 (segment (start 92 65) (end 146.976685 65) (width 0.2) (layer "F.Cu") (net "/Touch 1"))
 (segment (start 158.649 53.327685) (end 158.649 51.818786) (width 0.2) (layer "F.Cu") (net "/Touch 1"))
 (segment (start 74.5 90.5) (end 74.5 82.5) (width 0.2) (layer "F.Cu") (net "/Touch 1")))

